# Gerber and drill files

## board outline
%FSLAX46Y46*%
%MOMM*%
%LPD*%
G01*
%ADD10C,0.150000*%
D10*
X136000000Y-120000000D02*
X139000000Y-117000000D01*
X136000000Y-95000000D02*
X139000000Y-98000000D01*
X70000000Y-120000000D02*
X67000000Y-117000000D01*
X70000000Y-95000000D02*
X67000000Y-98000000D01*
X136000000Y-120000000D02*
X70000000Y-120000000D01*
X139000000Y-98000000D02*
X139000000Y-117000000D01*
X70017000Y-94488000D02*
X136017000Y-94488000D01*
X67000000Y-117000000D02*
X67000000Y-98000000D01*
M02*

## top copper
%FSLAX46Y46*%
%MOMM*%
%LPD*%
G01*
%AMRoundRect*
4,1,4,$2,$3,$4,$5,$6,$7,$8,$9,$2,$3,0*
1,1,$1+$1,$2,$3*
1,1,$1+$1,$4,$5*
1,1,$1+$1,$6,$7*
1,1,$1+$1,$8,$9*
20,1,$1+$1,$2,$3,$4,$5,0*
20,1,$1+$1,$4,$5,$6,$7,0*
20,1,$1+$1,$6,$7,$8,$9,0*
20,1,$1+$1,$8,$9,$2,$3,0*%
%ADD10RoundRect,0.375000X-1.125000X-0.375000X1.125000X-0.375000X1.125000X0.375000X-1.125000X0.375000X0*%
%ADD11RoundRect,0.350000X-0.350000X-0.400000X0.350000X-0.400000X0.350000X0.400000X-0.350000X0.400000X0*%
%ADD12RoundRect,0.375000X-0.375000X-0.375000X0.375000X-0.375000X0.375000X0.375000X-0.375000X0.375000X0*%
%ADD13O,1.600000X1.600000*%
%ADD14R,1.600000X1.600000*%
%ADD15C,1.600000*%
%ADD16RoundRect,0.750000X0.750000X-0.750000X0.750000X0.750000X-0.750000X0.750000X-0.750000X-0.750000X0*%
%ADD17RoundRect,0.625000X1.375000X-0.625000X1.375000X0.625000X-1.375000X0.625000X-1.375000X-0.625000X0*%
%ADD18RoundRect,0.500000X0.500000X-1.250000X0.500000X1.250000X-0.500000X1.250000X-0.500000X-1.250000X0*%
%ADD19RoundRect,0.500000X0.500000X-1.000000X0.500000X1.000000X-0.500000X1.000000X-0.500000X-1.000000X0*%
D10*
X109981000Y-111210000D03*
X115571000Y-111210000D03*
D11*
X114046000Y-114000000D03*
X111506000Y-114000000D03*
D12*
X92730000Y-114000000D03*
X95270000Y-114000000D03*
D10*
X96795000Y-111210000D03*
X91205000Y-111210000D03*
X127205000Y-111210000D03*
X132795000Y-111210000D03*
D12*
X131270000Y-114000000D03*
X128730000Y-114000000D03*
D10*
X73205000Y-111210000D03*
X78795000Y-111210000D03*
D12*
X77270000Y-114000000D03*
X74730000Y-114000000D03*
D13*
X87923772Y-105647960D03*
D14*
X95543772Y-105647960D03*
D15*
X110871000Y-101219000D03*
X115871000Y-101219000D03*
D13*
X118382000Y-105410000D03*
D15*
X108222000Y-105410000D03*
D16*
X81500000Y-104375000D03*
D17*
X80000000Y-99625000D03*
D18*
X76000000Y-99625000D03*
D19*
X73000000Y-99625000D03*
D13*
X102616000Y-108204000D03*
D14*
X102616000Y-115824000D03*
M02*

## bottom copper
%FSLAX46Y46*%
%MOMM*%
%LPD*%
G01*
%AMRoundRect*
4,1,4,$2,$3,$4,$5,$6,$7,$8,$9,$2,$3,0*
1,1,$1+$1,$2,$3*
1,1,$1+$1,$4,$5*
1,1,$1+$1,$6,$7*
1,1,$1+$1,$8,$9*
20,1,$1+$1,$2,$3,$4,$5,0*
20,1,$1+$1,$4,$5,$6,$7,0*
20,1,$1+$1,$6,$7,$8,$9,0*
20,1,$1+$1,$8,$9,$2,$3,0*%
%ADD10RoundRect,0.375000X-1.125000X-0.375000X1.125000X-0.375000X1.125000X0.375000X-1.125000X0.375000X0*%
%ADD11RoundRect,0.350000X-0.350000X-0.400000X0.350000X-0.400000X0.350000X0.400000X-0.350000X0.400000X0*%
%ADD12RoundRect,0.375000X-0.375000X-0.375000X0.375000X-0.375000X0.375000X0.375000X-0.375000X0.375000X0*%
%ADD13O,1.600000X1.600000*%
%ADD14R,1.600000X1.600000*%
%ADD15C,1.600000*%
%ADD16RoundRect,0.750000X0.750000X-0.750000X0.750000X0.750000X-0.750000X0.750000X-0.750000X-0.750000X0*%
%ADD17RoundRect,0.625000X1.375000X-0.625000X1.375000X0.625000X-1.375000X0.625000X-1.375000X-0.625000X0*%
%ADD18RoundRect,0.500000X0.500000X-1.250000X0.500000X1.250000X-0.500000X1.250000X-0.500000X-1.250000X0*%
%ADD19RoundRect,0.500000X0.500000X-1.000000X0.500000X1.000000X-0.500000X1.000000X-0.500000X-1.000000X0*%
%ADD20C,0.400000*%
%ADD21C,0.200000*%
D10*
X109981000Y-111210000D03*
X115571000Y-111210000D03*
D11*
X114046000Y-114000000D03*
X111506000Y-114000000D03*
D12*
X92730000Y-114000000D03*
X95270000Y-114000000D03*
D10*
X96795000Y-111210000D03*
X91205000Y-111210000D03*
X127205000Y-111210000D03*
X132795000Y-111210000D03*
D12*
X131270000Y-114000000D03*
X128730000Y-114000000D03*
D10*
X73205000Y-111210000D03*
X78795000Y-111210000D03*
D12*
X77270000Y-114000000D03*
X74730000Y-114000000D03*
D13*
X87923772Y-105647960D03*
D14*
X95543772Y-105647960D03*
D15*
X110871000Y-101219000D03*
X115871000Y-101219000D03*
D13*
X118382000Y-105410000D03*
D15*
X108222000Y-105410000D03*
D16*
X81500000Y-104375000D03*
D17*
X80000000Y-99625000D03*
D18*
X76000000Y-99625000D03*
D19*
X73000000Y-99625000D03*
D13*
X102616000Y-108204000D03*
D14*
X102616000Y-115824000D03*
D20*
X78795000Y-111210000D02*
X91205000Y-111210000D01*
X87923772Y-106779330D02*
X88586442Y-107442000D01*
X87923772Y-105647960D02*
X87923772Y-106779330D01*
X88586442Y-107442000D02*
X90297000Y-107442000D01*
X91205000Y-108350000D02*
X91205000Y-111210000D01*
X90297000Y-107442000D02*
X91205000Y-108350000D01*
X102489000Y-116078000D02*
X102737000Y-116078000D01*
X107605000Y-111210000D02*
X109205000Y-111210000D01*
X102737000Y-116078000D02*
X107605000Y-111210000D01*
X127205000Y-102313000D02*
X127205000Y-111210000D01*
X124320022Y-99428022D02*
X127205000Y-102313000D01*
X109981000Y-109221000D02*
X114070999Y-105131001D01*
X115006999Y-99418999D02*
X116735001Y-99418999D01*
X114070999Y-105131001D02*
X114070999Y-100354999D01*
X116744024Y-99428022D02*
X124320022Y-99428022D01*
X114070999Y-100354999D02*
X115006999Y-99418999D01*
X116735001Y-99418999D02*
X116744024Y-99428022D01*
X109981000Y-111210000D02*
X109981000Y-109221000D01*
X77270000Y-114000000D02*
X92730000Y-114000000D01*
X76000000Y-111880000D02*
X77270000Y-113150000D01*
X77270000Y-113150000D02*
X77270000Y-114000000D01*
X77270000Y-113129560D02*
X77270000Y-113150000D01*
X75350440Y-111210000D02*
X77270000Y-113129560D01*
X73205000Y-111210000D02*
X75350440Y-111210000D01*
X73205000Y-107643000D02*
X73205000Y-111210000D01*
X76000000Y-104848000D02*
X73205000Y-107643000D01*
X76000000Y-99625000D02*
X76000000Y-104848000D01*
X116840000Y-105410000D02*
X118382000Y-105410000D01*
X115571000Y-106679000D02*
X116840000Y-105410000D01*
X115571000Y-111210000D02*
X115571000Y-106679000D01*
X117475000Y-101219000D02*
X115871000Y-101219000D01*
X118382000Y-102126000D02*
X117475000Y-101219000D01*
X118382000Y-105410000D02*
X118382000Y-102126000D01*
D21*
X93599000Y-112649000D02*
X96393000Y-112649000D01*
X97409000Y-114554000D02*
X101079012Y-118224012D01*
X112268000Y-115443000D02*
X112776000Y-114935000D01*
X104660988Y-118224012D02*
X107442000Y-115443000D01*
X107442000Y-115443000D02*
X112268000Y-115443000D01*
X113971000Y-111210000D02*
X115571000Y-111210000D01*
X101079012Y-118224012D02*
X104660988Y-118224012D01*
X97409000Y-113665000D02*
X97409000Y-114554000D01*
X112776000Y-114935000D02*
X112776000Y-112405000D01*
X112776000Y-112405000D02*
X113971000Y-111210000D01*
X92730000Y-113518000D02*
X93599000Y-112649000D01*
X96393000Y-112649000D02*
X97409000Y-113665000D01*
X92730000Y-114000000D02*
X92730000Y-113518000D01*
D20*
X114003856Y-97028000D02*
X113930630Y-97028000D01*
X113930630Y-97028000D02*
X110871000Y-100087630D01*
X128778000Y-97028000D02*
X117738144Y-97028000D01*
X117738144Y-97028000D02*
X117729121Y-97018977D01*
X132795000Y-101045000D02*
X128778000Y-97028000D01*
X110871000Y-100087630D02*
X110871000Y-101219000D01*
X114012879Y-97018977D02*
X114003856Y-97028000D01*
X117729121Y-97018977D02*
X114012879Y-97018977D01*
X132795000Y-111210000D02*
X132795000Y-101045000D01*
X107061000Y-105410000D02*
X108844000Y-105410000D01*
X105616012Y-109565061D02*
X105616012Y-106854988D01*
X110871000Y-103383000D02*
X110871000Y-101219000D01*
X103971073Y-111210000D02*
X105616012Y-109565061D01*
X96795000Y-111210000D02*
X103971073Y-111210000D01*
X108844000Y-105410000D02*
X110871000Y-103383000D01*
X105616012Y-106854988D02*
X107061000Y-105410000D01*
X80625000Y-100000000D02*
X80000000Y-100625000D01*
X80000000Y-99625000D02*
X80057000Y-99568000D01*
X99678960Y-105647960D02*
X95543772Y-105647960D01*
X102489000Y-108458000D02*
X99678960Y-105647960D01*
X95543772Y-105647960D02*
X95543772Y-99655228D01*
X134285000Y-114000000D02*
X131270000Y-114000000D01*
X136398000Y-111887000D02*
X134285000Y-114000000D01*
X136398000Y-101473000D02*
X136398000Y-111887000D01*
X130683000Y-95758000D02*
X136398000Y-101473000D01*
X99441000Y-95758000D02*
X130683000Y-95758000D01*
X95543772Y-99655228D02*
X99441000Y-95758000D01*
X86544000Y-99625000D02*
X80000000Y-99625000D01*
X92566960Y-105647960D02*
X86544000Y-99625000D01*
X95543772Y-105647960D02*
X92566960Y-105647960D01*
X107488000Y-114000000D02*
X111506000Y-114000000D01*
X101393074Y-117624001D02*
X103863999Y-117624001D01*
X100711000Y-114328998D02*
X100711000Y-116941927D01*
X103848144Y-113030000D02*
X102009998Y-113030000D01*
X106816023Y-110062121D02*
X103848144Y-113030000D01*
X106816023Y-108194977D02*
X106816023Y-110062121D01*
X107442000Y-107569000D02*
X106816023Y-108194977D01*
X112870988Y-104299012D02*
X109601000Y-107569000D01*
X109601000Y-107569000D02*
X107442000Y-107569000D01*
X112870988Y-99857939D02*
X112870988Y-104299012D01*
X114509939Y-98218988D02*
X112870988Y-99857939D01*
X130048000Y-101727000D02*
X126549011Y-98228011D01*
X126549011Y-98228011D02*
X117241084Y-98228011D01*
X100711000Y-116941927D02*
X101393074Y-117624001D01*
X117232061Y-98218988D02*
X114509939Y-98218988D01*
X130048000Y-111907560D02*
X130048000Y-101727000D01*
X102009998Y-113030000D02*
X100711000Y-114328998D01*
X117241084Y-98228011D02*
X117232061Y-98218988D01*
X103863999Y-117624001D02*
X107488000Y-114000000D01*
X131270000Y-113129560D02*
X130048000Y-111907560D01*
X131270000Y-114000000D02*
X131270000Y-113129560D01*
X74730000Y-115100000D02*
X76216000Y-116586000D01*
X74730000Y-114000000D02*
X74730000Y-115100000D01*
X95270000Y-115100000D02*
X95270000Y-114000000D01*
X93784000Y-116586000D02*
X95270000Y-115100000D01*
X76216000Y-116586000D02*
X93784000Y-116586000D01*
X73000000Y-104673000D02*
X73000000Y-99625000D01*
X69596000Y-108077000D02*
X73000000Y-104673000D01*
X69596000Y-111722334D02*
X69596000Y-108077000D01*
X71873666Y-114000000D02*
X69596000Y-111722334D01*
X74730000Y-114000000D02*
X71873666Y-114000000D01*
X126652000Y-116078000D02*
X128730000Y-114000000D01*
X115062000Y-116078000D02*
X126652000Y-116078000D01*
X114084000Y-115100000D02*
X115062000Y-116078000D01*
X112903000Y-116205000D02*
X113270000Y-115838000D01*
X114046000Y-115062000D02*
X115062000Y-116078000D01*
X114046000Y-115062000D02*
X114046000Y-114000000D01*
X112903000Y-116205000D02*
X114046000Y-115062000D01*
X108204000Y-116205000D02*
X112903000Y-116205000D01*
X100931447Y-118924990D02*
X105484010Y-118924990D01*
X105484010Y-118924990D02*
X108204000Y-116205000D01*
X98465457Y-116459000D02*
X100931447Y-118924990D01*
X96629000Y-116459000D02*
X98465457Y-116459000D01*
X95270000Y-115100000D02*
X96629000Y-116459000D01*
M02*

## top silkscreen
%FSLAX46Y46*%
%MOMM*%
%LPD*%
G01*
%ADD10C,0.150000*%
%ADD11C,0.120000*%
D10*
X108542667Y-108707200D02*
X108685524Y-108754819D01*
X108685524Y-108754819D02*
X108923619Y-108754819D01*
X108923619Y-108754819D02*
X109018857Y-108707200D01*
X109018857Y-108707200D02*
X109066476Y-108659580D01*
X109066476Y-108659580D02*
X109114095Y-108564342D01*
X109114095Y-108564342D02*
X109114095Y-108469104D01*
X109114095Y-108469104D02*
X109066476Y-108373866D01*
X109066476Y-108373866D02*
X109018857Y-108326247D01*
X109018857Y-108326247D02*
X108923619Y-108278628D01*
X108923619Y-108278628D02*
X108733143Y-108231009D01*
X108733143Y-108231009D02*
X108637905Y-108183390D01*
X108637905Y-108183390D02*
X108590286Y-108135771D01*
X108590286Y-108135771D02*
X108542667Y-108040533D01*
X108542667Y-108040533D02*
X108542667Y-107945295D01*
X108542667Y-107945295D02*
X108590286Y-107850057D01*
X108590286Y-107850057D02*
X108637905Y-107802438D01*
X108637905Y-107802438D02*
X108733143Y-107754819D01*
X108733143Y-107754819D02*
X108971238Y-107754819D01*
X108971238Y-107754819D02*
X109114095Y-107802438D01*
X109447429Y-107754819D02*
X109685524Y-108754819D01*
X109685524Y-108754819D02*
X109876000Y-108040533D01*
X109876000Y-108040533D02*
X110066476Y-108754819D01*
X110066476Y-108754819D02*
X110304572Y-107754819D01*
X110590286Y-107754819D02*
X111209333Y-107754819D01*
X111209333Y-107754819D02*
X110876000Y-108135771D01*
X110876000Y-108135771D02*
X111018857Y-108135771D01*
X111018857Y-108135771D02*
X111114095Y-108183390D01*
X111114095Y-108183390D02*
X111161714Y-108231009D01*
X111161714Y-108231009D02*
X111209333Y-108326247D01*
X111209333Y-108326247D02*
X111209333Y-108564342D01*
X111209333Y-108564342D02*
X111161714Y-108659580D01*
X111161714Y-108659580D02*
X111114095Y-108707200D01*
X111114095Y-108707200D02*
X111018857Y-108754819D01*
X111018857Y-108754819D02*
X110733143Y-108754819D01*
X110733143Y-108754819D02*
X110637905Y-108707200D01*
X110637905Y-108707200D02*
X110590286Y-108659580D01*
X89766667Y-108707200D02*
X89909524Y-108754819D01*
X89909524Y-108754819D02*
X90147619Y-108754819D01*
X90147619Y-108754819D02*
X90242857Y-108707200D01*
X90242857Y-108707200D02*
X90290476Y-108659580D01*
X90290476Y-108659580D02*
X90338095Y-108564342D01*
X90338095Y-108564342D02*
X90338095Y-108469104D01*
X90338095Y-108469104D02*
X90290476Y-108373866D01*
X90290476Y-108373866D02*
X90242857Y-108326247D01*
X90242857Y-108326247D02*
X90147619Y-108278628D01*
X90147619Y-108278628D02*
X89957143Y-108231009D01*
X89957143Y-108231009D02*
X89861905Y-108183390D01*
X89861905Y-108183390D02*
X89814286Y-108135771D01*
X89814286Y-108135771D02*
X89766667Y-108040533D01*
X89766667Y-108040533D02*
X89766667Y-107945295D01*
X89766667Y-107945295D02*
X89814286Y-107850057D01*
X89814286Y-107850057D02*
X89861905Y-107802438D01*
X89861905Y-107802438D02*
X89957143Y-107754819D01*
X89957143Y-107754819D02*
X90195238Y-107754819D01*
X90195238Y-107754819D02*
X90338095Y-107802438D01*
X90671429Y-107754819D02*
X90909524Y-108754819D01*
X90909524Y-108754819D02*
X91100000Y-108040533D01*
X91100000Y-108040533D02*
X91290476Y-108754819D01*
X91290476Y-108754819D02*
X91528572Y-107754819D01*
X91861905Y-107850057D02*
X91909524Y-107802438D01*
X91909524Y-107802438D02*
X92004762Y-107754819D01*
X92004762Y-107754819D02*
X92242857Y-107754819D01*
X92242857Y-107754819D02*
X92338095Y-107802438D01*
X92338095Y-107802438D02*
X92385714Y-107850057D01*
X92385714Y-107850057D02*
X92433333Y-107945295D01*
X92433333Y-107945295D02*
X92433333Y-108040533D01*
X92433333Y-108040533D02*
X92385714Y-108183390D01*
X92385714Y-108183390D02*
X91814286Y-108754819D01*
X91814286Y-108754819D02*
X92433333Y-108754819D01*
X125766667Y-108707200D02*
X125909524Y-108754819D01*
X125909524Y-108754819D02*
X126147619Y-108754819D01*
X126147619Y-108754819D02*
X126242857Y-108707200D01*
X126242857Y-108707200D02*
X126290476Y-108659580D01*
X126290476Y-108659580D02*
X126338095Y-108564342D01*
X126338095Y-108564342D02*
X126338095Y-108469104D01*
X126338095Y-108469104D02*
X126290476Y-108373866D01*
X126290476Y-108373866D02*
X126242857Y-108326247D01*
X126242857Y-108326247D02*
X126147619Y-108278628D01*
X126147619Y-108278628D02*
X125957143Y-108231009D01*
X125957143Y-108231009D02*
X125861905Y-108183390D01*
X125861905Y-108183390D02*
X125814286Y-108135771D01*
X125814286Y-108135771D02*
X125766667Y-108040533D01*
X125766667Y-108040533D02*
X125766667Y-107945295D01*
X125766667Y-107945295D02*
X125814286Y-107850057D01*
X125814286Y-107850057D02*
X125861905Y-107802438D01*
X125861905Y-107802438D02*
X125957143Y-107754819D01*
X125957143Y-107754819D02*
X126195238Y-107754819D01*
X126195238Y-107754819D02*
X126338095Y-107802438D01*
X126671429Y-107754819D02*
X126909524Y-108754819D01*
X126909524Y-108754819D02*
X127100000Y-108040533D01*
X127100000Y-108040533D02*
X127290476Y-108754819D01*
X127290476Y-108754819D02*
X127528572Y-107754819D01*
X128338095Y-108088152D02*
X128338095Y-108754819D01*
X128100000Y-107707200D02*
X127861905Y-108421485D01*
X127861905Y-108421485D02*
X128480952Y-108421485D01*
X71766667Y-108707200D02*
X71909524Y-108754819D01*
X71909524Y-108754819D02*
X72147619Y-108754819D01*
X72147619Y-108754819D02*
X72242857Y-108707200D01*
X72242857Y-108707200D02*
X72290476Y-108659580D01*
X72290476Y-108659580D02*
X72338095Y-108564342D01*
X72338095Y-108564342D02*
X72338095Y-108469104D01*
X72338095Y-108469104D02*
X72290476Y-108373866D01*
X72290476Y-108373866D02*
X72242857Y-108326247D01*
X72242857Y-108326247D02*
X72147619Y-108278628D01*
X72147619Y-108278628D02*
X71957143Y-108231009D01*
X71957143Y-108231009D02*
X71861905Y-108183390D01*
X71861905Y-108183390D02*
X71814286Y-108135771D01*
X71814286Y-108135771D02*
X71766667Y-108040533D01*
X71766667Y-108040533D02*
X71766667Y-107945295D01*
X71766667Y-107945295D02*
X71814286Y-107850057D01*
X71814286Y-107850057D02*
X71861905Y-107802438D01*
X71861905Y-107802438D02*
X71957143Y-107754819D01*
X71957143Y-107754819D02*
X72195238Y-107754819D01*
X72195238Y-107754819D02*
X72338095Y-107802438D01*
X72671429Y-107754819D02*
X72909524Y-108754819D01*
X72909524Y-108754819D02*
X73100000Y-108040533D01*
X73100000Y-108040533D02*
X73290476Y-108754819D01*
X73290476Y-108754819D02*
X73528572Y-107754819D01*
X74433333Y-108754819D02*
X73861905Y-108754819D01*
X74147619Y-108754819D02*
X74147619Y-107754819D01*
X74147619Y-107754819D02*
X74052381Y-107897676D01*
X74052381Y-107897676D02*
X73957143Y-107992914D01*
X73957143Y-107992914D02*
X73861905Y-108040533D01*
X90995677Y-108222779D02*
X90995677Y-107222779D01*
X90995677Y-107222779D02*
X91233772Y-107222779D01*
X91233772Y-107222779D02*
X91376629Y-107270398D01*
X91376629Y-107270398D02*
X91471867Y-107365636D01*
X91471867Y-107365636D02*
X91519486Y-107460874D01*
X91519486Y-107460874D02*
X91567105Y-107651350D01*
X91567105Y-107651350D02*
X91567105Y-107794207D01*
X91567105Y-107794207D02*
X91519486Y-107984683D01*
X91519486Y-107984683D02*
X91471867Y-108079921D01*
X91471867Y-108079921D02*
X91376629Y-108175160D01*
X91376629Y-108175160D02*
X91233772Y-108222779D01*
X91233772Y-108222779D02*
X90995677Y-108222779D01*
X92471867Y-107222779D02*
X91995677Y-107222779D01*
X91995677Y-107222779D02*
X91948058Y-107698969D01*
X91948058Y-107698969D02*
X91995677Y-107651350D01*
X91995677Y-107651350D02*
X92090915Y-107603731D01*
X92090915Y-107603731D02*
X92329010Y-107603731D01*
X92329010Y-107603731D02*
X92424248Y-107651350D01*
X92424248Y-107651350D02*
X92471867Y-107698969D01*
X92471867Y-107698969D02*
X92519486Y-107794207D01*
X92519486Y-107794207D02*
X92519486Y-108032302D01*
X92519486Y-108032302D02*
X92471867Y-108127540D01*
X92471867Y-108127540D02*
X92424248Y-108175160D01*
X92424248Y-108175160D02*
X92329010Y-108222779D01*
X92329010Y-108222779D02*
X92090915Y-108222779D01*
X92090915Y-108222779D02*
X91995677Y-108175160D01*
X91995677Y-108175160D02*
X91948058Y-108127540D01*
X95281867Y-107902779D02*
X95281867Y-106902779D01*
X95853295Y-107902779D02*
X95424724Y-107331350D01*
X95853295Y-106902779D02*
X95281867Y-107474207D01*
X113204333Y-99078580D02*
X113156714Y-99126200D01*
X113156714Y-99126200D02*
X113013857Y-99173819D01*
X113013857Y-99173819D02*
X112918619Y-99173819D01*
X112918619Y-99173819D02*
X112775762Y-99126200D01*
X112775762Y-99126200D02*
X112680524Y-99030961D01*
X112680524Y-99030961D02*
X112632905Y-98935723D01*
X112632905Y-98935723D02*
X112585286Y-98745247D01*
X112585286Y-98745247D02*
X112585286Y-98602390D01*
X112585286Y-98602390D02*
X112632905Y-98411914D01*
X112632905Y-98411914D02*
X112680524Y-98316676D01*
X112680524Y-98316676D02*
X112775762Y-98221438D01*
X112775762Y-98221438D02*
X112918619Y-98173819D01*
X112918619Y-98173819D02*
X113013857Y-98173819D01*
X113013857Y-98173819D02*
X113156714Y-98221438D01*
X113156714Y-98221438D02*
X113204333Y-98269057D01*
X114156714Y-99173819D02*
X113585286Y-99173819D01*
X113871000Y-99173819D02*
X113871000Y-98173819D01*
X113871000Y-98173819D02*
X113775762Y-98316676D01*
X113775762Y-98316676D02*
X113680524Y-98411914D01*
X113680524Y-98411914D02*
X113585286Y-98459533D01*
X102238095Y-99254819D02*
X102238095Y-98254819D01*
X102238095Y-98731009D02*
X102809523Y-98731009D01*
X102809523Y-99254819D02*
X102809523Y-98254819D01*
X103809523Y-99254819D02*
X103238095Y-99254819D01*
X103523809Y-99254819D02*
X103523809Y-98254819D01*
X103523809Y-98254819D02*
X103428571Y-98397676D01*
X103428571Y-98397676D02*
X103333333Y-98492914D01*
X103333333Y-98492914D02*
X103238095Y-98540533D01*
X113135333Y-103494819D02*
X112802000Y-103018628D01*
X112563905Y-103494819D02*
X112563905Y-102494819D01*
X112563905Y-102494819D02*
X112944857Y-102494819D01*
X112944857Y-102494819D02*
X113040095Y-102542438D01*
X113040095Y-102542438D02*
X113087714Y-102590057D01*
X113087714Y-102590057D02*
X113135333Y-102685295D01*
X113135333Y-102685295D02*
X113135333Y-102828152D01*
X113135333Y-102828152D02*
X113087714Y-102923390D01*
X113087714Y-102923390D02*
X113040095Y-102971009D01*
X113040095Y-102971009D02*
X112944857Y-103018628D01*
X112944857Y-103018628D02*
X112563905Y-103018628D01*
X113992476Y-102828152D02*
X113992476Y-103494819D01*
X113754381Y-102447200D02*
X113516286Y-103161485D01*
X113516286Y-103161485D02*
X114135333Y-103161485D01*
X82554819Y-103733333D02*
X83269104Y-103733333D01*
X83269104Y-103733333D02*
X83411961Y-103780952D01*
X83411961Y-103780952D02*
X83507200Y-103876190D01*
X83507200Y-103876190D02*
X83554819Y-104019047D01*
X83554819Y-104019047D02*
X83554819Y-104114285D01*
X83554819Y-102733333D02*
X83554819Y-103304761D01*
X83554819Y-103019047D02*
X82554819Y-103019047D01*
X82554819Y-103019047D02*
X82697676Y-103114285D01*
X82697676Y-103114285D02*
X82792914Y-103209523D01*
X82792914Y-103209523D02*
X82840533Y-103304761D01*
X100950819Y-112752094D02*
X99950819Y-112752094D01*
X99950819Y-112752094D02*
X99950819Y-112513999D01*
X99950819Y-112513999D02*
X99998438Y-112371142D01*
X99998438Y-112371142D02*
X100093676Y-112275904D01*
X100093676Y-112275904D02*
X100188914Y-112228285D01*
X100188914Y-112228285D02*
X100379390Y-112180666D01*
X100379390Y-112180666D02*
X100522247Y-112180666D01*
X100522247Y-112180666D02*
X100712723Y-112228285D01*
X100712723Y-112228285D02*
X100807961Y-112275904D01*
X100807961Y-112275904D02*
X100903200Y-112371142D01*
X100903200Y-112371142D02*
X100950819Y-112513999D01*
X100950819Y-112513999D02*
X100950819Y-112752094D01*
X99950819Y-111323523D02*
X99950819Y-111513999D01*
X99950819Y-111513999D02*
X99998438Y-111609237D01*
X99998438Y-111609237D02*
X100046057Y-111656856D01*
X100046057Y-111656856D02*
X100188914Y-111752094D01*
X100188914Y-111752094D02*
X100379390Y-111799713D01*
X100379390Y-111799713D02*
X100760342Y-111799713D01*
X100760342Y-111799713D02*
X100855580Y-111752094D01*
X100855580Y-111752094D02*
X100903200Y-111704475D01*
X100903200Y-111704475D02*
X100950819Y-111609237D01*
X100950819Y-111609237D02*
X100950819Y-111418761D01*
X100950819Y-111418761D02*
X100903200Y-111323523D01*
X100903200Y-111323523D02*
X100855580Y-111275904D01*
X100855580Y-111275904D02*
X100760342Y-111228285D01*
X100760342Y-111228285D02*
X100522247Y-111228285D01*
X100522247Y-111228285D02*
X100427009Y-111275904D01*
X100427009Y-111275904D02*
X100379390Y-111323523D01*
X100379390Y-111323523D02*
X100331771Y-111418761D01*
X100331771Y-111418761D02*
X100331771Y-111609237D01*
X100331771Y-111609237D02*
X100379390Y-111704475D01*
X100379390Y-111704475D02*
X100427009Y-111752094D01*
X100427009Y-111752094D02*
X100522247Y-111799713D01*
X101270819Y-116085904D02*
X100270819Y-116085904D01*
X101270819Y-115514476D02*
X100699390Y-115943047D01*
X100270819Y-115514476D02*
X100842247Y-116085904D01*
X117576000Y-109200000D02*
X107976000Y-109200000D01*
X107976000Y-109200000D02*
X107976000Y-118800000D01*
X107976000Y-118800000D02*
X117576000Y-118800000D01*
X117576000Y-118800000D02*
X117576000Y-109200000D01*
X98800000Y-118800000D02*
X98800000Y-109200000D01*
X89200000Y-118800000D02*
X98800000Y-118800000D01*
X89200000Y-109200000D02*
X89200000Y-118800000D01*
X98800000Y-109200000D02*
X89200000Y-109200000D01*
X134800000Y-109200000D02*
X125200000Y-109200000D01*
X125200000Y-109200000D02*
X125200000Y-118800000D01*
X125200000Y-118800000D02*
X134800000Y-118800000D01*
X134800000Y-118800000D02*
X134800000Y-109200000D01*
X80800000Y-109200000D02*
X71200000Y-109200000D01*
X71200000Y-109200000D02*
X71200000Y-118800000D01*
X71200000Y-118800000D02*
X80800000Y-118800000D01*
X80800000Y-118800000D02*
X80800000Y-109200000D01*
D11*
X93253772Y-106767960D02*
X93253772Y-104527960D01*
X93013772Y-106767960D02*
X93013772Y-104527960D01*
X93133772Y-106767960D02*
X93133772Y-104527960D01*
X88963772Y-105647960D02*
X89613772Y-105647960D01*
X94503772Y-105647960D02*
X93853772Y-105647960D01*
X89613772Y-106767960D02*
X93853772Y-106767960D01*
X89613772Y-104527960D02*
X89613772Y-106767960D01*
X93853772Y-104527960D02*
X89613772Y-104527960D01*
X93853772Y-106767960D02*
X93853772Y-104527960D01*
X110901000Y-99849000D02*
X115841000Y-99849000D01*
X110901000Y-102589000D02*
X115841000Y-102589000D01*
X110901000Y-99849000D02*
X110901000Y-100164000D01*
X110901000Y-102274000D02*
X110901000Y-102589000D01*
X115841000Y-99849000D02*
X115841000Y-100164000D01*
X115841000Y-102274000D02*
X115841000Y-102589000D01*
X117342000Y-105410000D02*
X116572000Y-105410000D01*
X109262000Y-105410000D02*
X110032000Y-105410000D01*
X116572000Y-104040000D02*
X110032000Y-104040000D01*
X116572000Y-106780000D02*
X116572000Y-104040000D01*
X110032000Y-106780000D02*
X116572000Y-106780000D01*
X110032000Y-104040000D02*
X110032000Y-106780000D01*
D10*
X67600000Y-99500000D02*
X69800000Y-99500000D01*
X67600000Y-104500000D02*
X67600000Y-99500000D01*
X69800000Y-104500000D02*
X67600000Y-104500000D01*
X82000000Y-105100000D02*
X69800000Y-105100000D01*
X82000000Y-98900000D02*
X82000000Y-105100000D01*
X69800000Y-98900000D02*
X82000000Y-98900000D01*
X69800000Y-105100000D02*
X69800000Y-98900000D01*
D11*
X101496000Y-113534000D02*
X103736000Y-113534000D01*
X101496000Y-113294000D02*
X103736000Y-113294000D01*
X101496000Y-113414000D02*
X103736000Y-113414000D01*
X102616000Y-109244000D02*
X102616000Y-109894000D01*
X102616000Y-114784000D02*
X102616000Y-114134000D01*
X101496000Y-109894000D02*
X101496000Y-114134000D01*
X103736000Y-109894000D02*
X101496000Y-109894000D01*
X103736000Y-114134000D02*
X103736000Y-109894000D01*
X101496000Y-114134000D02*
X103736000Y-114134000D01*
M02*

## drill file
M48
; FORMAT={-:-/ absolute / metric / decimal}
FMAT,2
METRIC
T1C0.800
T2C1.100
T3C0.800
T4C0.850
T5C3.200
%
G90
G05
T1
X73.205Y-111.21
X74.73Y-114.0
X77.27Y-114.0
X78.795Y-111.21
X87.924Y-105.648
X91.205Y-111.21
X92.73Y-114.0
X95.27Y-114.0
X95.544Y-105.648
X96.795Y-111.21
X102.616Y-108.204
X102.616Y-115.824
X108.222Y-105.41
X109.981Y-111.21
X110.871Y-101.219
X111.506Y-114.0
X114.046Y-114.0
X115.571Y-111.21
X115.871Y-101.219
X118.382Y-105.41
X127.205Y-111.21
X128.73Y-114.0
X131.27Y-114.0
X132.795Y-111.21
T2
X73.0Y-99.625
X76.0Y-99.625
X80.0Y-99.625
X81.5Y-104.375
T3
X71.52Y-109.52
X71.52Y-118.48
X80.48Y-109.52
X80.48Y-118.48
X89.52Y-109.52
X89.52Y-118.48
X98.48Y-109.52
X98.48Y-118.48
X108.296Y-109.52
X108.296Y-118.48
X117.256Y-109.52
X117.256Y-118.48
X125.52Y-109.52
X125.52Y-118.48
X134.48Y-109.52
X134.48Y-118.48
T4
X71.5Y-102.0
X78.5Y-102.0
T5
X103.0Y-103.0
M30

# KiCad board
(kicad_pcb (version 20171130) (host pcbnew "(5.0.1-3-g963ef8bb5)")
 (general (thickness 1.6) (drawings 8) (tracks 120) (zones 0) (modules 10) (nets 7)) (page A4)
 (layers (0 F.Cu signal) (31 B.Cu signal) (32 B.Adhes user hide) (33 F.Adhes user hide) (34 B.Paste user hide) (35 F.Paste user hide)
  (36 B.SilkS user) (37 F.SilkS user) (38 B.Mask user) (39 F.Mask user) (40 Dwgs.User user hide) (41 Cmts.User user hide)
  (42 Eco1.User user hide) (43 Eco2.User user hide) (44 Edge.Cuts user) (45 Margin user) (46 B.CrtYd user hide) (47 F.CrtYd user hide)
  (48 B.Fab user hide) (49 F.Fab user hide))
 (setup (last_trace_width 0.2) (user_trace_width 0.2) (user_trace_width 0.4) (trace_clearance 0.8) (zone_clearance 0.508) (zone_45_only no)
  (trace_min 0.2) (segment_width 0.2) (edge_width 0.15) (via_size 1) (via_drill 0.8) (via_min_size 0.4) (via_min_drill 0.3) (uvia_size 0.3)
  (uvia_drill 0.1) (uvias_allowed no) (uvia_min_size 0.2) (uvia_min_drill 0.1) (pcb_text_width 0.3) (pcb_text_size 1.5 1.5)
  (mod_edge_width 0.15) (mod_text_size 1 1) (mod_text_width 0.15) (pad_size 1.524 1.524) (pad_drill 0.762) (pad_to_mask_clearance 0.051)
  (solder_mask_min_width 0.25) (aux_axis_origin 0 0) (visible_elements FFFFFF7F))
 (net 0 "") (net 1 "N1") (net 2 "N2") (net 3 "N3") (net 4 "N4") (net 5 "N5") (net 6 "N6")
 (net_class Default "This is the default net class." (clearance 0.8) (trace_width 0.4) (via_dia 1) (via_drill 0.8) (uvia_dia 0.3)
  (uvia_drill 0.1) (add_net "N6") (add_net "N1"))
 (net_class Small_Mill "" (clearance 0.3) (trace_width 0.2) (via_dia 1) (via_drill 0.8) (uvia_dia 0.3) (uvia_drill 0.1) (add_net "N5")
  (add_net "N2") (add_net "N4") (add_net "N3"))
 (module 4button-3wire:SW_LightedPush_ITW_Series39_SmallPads (layer F.Cu) (at 112.776 114)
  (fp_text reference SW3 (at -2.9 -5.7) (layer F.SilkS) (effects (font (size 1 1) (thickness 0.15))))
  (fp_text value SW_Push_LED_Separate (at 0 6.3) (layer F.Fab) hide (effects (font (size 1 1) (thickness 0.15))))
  (fp_line (start 4.8 -4.8) (end -4.8 -4.8) (layer F.SilkS) (width 0.15))
  (fp_line (start -4.8 -4.8) (end -4.8 4.8) (layer F.SilkS) (width 0.15))
  (fp_line (start -4.8 4.8) (end 4.8 4.8) (layer F.SilkS) (width 0.15))
  (fp_line (start 4.8 4.8) (end 4.8 -4.8) (layer F.SilkS) (width 0.15))
  (pad 1 thru_hole roundrect (at -2.795 -2.79) (size 3 1.5) (drill 0.8) (layers *.Cu *.Mask) (roundrect_rratio 0.25) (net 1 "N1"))
  (pad 2 thru_hole roundrect (at 2.795 -2.79) (size 3 1.5) (drill 0.8) (layers *.Cu *.Mask) (roundrect_rratio 0.25) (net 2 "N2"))
  (pad 3 thru_hole roundrect (at 1.27 0) (size 1.4 1.5) (drill 0.8) (layers *.Cu *.Mask) (roundrect_rratio 0.25) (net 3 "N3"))
  (pad 4 thru_hole roundrect (at -1.27 0) (size 1.4 1.5) (drill 0.8) (layers *.Cu *.Mask) (roundrect_rratio 0.25) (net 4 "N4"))
  (pad "" np_thru_hole circle (at 4.48 4.48) (size 0.8 0.8) (drill 0.8) (layers *.Cu *.Mask))
  (pad "" np_thru_hole circle (at -4.48 4.48) (size 0.8 0.8) (drill 0.8) (layers *.Cu *.Mask))
  (pad "" np_thru_hole circle (at 4.48 -4.48) (size 0.8 0.8) (drill 0.8) (layers *.Cu *.Mask))
  (pad "" np_thru_hole circle (at -4.48 -4.48) (size 0.8 0.8) (drill 0.8) (layers *.Cu *.Mask)))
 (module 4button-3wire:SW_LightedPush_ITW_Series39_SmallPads (layer F.Cu) (at 94 114)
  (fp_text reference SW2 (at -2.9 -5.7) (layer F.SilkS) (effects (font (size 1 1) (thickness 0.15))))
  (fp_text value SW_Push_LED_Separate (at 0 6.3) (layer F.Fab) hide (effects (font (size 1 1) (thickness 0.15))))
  (fp_line (start 4.8 4.8) (end 4.8 -4.8) (layer F.SilkS) (width 0.15))
  (fp_line (start -4.8 4.8) (end 4.8 4.8) (layer F.SilkS) (width 0.15))
  (fp_line (start -4.8 -4.8) (end -4.8 4.8) (layer F.SilkS) (width 0.15))
  (fp_line (start 4.8 -4.8) (end -4.8 -4.8) (layer F.SilkS) (width 0.15))
  (pad "" np_thru_hole circle (at -4.48 -4.48) (size 0.8 0.8) (drill 0.8) (layers *.Cu *.Mask))
  (pad "" np_thru_hole circle (at 4.48 -4.48) (size 0.8 0.8) (drill 0.8) (layers *.Cu *.Mask))
  (pad "" np_thru_hole circle (at -4.48 4.48) (size 0.8 0.8) (drill 0.8) (layers *.Cu *.Mask))
  (pad "" np_thru_hole circle (at 4.48 4.48) (size 0.8 0.8) (drill 0.8) (layers *.Cu *.Mask))
  (pad 4 thru_hole roundrect (at -1.27 0) (size 1.5 1.5) (drill 0.8) (layers *.Cu *.Mask) (roundrect_rratio 0.25) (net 2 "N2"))
  (pad 3 thru_hole roundrect (at 1.27 0) (size 1.5 1.5) (drill 0.8) (layers *.Cu *.Mask) (roundrect_rratio 0.25) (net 3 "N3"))
  (pad 2 thru_hole roundrect (at 2.795 -2.79) (size 3 1.5) (drill 0.8) (layers *.Cu *.Mask) (roundrect_rratio 0.25) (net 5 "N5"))
  (pad 1 thru_hole roundrect (at -2.795 -2.79) (size 3 1.5) (drill 0.8) (layers *.Cu *.Mask) (roundrect_rratio 0.25) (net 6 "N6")))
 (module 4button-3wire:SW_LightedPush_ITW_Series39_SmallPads (layer F.Cu) (at 130 114)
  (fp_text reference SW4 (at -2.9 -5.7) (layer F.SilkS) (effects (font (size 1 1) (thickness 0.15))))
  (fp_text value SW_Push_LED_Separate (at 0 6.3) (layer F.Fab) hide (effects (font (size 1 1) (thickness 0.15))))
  (fp_line (start 4.8 -4.8) (end -4.8 -4.8) (layer F.SilkS) (width 0.15))
  (fp_line (start -4.8 -4.8) (end -4.8 4.8) (layer F.SilkS) (width 0.15))
  (fp_line (start -4.8 4.8) (end 4.8 4.8) (layer F.SilkS) (width 0.15))
  (fp_line (start 4.8 4.8) (end 4.8 -4.8) (layer F.SilkS) (width 0.15))
  (pad 1 thru_hole roundrect (at -2.795 -2.79) (size 3 1.5) (drill 0.8) (layers *.Cu *.Mask) (roundrect_rratio 0.25) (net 1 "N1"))
  (pad 2 thru_hole roundrect (at 2.795 -2.79) (size 3 1.5) (drill 0.8) (layers *.Cu *.Mask) (roundrect_rratio 0.25) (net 5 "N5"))
  (pad 3 thru_hole roundrect (at 1.27 0) (size 1.5 1.5) (drill 0.8) (layers *.Cu *.Mask) (roundrect_rratio 0.25) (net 4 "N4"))
  (pad 4 thru_hole roundrect (at -1.27 0) (size 1.5 1.5) (drill 0.8) (layers *.Cu *.Mask) (roundrect_rratio 0.25) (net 3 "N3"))
  (pad "" np_thru_hole circle (at 4.48 4.48) (size 0.8 0.8) (drill 0.8) (layers *.Cu *.Mask))
  (pad "" np_thru_hole circle (at -4.48 4.48) (size 0.8 0.8) (drill 0.8) (layers *.Cu *.Mask))
  (pad "" np_thru_hole circle (at 4.48 -4.48) (size 0.8 0.8) (drill 0.8) (layers *.Cu *.Mask))
  (pad "" np_thru_hole circle (at -4.48 -4.48) (size 0.8 0.8) (drill 0.8) (layers *.Cu *.Mask)))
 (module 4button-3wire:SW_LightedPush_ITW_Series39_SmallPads (layer F.Cu) (at 76 114)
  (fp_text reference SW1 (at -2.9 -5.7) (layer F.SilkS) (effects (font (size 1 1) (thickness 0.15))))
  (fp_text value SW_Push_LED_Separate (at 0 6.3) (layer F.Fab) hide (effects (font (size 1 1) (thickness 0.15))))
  (fp_line (start 4.8 -4.8) (end -4.8 -4.8) (layer F.SilkS) (width 0.15))
  (fp_line (start -4.8 -4.8) (end -4.8 4.8) (layer F.SilkS) (width 0.15))
  (fp_line (start -4.8 4.8) (end 4.8 4.8) (layer F.SilkS) (width 0.15))
  (fp_line (start 4.8 4.8) (end 4.8 -4.8) (layer F.SilkS) (width 0.15))
  (pad 1 thru_hole roundrect (at -2.795 -2.79) (size 3 1.5) (drill 0.8) (layers *.Cu *.Mask) (roundrect_rratio 0.25) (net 2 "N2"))
  (pad 2 thru_hole roundrect (at 2.795 -2.79) (size 3 1.5) (drill 0.8) (layers *.Cu *.Mask) (roundrect_rratio 0.25) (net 6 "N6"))
  (pad 3 thru_hole roundrect (at 1.27 0) (size 1.5 1.5) (drill 0.8) (layers *.Cu *.Mask) (roundrect_rratio 0.25) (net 2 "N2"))
  (pad 4 thru_hole roundrect (at -1.27 0) (size 1.5 1.5) (drill 0.8) (layers *.Cu *.Mask) (roundrect_rratio 0.25) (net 3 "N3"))
  (pad "" np_thru_hole circle (at 4.48 4.48) (size 0.8 0.8) (drill 0.8) (layers *.Cu *.Mask))
  (pad "" np_thru_hole circle (at -4.48 4.48) (size 0.8 0.8) (drill 0.8) (layers *.Cu *.Mask))
  (pad "" np_thru_hole circle (at 4.48 -4.48) (size 0.8 0.8) (drill 0.8) (layers *.Cu *.Mask))
  (pad "" np_thru_hole circle (at -4.48 -4.48) (size 0.8 0.8) (drill 0.8) (layers *.Cu *.Mask)))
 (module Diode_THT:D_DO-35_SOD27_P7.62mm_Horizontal (layer F.Cu) (at 95.543772 105.64796 180)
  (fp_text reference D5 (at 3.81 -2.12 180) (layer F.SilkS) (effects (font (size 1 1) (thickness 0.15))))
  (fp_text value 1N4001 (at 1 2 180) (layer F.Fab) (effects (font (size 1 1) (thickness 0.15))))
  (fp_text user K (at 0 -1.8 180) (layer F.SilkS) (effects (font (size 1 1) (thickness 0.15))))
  (fp_line (start 2.29 -1.12) (end 2.29 1.12) (layer F.SilkS) (width 0.12))
  (fp_line (start 2.53 -1.12) (end 2.53 1.12) (layer F.SilkS) (width 0.12))
  (fp_line (start 2.41 -1.12) (end 2.41 1.12) (layer F.SilkS) (width 0.12))
  (fp_line (start 6.58 0) (end 5.93 0) (layer F.SilkS) (width 0.12))
  (fp_line (start 1.04 0) (end 1.69 0) (layer F.SilkS) (width 0.12))
  (fp_line (start 5.93 -1.12) (end 1.69 -1.12) (layer F.SilkS) (width 0.12))
  (fp_line (start 5.93 1.12) (end 5.93 -1.12) (layer F.SilkS) (width 0.12))
  (fp_line (start 1.69 1.12) (end 5.93 1.12) (layer F.SilkS) (width 0.12))
  (fp_line (start 1.69 -1.12) (end 1.69 1.12) (layer F.SilkS) (width 0.12))
  (pad 2 thru_hole oval (at 7.62 0 180) (size 1.6 1.6) (drill 0.8) (layers *.Cu *.Mask) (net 6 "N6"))
  (pad 1 thru_hole rect (at 0 0 180) (size 1.6 1.6) (drill 0.8) (layers *.Cu *.Mask) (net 4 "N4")))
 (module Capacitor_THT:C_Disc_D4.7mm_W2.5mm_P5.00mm (layer F.Cu) (at 110.871 101.219)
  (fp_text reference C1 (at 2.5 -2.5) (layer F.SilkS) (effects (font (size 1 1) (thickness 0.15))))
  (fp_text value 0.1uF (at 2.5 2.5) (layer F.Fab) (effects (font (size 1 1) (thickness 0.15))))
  (fp_line (start 0.03 -1.37) (end 4.97 -1.37) (layer F.SilkS) (width 0.12))
  (fp_line (start 0.03 1.37) (end 4.97 1.37) (layer F.SilkS) (width 0.12))
  (fp_line (start 0.03 -1.37) (end 0.03 -1.055) (layer F.SilkS) (width 0.12))
  (fp_line (start 0.03 1.055) (end 0.03 1.37) (layer F.SilkS) (width 0.12))
  (fp_line (start 4.97 -1.37) (end 4.97 -1.055) (layer F.SilkS) (width 0.12))
  (fp_line (start 4.97 1.055) (end 4.97 1.37) (layer F.SilkS) (width 0.12))
  (pad 1 thru_hole circle (at 0 0) (size 1.6 1.6) (drill 0.8) (layers *.Cu *.Mask) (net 5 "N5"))
  (pad 2 thru_hole circle (at 5 0) (size 1.6 1.6) (drill 0.8) (layers *.Cu *.Mask) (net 2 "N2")))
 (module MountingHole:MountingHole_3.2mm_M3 (layer F.Cu) (at 103 103)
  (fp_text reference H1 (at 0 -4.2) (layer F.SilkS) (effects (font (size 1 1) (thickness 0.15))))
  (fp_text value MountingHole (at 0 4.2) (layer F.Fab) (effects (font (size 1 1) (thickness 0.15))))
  (pad 1 np_thru_hole circle (at 0 0) (size 3.2 3.2) (drill 3.2) (layers *.Cu *.Mask)))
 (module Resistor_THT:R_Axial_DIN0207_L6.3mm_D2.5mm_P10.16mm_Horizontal (layer F.Cu) (at 108.222 105.41)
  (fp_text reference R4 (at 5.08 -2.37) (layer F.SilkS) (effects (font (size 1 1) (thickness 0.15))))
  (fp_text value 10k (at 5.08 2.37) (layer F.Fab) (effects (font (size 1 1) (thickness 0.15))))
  (fp_line (start 9.12 0) (end 8.35 0) (layer F.SilkS) (width 0.12))
  (fp_line (start 1.04 0) (end 1.81 0) (layer F.SilkS) (width 0.12))
  (fp_line (start 8.35 -1.37) (end 1.81 -1.37) (layer F.SilkS) (width 0.12))
  (fp_line (start 8.35 1.37) (end 8.35 -1.37) (layer F.SilkS) (width 0.12))
  (fp_line (start 1.81 1.37) (end 8.35 1.37) (layer F.SilkS) (width 0.12))
  (fp_line (start 1.81 -1.37) (end 1.81 1.37) (layer F.SilkS) (width 0.12))
  (pad 2 thru_hole oval (at 10.16 0) (size 1.6 1.6) (drill 0.8) (layers *.Cu *.Mask) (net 2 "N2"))
  (pad 1 thru_hole circle (at 0 0) (size 1.6 1.6) (drill 0.8) (layers *.Cu *.Mask) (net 5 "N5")))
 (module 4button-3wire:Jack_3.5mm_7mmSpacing (layer F.Cu) (at 82 102 90)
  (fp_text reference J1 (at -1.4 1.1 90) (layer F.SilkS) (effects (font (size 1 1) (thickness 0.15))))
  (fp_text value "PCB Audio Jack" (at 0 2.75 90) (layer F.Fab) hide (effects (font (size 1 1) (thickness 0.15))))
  (fp_line (start 2.5 -14.4) (end 2.5 -12.2) (layer F.SilkS) (width 0.15))
  (fp_line (start -2.5 -14.4) (end 2.5 -14.4) (layer F.SilkS) (width 0.15))
  (fp_line (start -2.5 -12.2) (end -2.5 -14.4) (layer F.SilkS) (width 0.15))
  (fp_line (start -3.1 0) (end -3.1 -12.2) (layer F.SilkS) (width 0.15))
  (fp_line (start 3.1 0) (end -3.1 0) (layer F.SilkS) (width 0.15))
  (fp_line (start 3.1 -12.2) (end 3.1 0) (layer F.SilkS) (width 0.15))
  (fp_line (start -3.1 -12.2) (end 3.1 -12.2) (layer F.SilkS) (width 0.15))
  (pad "" np_thru_hole circle (at 0 -3.5 90) (size 0.85 0.85) (drill 0.85) (layers *.Cu *.Mask))
  (pad "" np_thru_hole circle (at 0 -10.5 90) (size 0.85 0.85) (drill 0.85) (layers *.Cu *.Mask))
  (pad X thru_hole roundrect (at -2.375 -0.5 90) (size 3 3) (drill 1.1) (layers *.Cu *.Mask) (roundrect_rratio 0.25))
  (pad T thru_hole roundrect (at 2.375 -2 90) (size 2.5 4) (drill 1.1) (layers *.Cu *.Mask) (roundrect_rratio 0.25) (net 4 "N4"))
  (pad R thru_hole roundrect (at 2.375 -6 90) (size 3.5 2) (drill 1.1) (layers *.Cu *.Mask) (roundrect_rratio 0.25) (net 2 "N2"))
  (pad S thru_hole roundrect (at 2.375 -9 90) (size 3 2) (drill 1.1) (layers *.Cu *.Mask) (roundrect_rratio 0.25) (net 3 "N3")))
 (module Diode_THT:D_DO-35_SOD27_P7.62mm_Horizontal (layer F.Cu) (at 102.616 115.824 90)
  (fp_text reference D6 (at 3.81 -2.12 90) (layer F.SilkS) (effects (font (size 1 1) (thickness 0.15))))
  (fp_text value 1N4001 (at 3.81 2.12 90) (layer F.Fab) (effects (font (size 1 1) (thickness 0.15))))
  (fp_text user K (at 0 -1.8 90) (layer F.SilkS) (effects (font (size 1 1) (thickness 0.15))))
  (fp_line (start 2.29 -1.12) (end 2.29 1.12) (layer F.SilkS) (width 0.12))
  (fp_line (start 2.53 -1.12) (end 2.53 1.12) (layer F.SilkS) (width 0.12))
  (fp_line (start 2.41 -1.12) (end 2.41 1.12) (layer F.SilkS) (width 0.12))
  (fp_line (start 6.58 0) (end 5.93 0) (layer F.SilkS) (width 0.12))
  (fp_line (start 1.04 0) (end 1.69 0) (layer F.SilkS) (width 0.12))
  (fp_line (start 5.93 -1.12) (end 1.69 -1.12) (layer F.SilkS) (width 0.12))
  (fp_line (start 5.93 1.12) (end 5.93 -1.12) (layer F.SilkS) (width 0.12))
  (fp_line (start 1.69 1.12) (end 5.93 1.12) (layer F.SilkS) (width 0.12))
  (fp_line (start 1.69 -1.12) (end 1.69 1.12) (layer F.SilkS) (width 0.12))
  (pad 2 thru_hole oval (at 7.62 0 90) (size 1.6 1.6) (drill 0.8) (layers *.Cu *.Mask) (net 4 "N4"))
  (pad 1 thru_hole rect (at 0 0 90) (size 1.6 1.6) (drill 0.8) (layers *.Cu *.Mask) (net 1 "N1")))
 (gr_line (start 136 120) (end 139 117) (layer Edge.Cuts) (width 0.15))
 (gr_line (start 136 95) (end 139 98) (layer Edge.Cuts) (width 0.15))
 (gr_line (start 70 120) (end 67 117) (layer Edge.Cuts) (width 0.15))
 (gr_line (start 70 95) (end 67 98) (layer Edge.Cuts) (width 0.15))
 (gr_line (start 136 120) (end 70 120) (layer Edge.Cuts) (width 0.15))
 (gr_line (start 139 98) (end 139 117) (layer Edge.Cuts) (width 0.15))
 (gr_line (start 70.017 94.488) (end 136.017 94.488) (layer Edge.Cuts) (width 0.15))
 (gr_line (start 67 117) (end 67 98) (layer Edge.Cuts) (width 0.15))
 (segment (start 78.795 111.21) (end 91.205 111.21) (width 0.4) (layer B.Cu) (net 6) (status 30))
 (segment (start 87.923772 106.77933) (end 88.586442 107.442) (width 0.4) (layer B.Cu) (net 6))
 (segment (start 87.923772 105.64796) (end 87.923772 106.77933) (width 0.4) (layer B.Cu) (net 6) (status 10))
 (segment (start 88.586442 107.442) (end 90.297 107.442) (width 0.4) (layer B.Cu) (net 6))
 (segment (start 91.205 108.35) (end 91.205 111.21) (width 0.4) (layer B.Cu) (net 6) (status 20))
 (segment (start 90.297 107.442) (end 91.205 108.35) (width 0.4) (layer B.Cu) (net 6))
 (segment (start 102.489 116.078) (end 102.737 116.078) (width 0.4) (layer B.Cu) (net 1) (status 30))
 (segment (start 107.605 111.21) (end 109.205 111.21) (width 0.4) (layer B.Cu) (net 1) (status 20))
 (segment (start 102.737 116.078) (end 107.605 111.21) (width 0.4) (layer B.Cu) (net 1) (status 10))
 (segment (start 127.205 102.313) (end 127.205 111.21) (width 0.4) (layer B.Cu) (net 1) (status 20))
 (segment (start 124.320022 99.428022) (end 127.205 102.313) (width 0.4) (layer B.Cu) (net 1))
 (segment (start 109.981 109.221) (end 114.070999 105.131001) (width 0.4) (layer B.Cu) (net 1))
 (segment (start 115.006999 99.418999) (end 116.735001 99.418999) (width 0.4) (layer B.Cu) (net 1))
 (segment (start 114.070999 105.131001) (end 114.070999 100.354999) (width 0.4) (layer B.Cu) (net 1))
 (segment (start 116.744024 99.428022) (end 124.320022 99.428022) (width 0.4) (layer B.Cu) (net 1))
 (segment (start 114.070999 100.354999) (end 115.006999 99.418999) (width 0.4) (layer B.Cu) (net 1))
 (segment (start 116.735001 99.418999) (end 116.744024 99.428022) (width 0.4) (layer B.Cu) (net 1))
 (segment (start 109.981 111.21) (end 109.981 109.221) (width 0.4) (layer B.Cu) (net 1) (status 10))
 (segment (start 77.27 114) (end 92.73 114) (width 0.4) (layer B.Cu) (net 2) (status 30))
 (segment (start 76 111.88) (end 77.27 113.15) (width 0.4) (layer B.Cu) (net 2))
 (segment (start 77.27 113.15) (end 77.27 114) (width 0.4) (layer B.Cu) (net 2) (status 20))
 (segment (start 77.27 113.12956) (end 77.27 113.15) (width 0.4) (layer B.Cu) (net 2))
 (segment (start 75.35044 111.21) (end 77.27 113.12956) (width 0.4) (layer B.Cu) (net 2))
 (segment (start 73.205 111.21) (end 75.35044 111.21) (width 0.4) (layer B.Cu) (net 2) (status 10))
 (segment (start 73.205 107.643) (end 73.205 111.21) (width 0.4) (layer B.Cu) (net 2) (status 20))
 (segment (start 76 104.848) (end 73.205 107.643) (width 0.4) (layer B.Cu) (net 2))
 (segment (start 76 99.625) (end 76 104.848) (width 0.4) (layer B.Cu) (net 2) (status 10))
 (segment (start 116.84 105.41) (end 118.382 105.41) (width 0.4) (layer B.Cu) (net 2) (status 20))
 (segment (start 115.571 106.679) (end 116.84 105.41) (width 0.4) (layer B.Cu) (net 2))
 (segment (start 115.571 111.21) (end 115.571 106.679) (width 0.4) (layer B.Cu) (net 2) (status 10))
 (segment (start 117.475 101.219) (end 115.871 101.219) (width 0.4) (layer B.Cu) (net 2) (status 20))
 (segment (start 118.382 102.126) (end 117.475 101.219) (width 0.4) (layer B.Cu) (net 2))
 (segment (start 118.382 105.41) (end 118.382 102.126) (width 0.4) (layer B.Cu) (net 2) (status 10))
 (segment (start 93.599 112.649) (end 96.393 112.649) (width 0.2) (layer B.Cu) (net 2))
 (segment (start 97.409 114.554) (end 101.079012 118.224012) (width 0.2) (layer B.Cu) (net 2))
 (segment (start 112.268 115.443) (end 112.776 114.935) (width 0.2) (layer B.Cu) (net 2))
 (segment (start 104.660988 118.224012) (end 107.442 115.443) (width 0.2) (layer B.Cu) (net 2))
 (segment (start 107.442 115.443) (end 112.268 115.443) (width 0.2) (layer B.Cu) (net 2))
 (segment (start 113.971 111.21) (end 115.571 111.21) (width 0.2) (layer B.Cu) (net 2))
 (segment (start 101.079012 118.224012) (end 104.660988 118.224012) (width 0.2) (layer B.Cu) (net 2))
 (segment (start 97.409 113.665) (end 97.409 114.554) (width 0.2) (layer B.Cu) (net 2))
 (segment (start 112.776 114.935) (end 112.776 112.405) (width 0.2) (layer B.Cu) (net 2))
 (segment (start 112.776 112.405) (end 113.971 111.21) (width 0.2) (layer B.Cu) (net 2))
 (segment (start 92.73 113.518) (end 93.599 112.649) (width 0.2) (layer B.Cu) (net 2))
 (segment (start 96.393 112.649) (end 97.409 113.665) (width 0.2) (layer B.Cu) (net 2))
 (segment (start 92.73 114) (end 92.73 113.518) (width 0.2) (layer B.Cu) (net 2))
 (segment (start 114.003856 97.028) (end 113.93063 97.028) (width 0.4) (layer B.Cu) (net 5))
 (segment (start 113.93063 97.028) (end 110.871 100.08763) (width 0.4) (layer B.Cu) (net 5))
 (segment (start 128.778 97.028) (end 117.738144 97.028) (width 0.4) (layer B.Cu) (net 5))
 (segment (start 117.738144 97.028) (end 117.729121 97.018977) (width 0.4) (layer B.Cu) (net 5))
 (segment (start 132.795 101.045) (end 128.778 97.028) (width 0.4) (layer B.Cu) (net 5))
 (segment (start 110.871 100.08763) (end 110.871 101.219) (width 0.4) (layer B.Cu) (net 5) (status 20))
 (segment (start 114.012879 97.018977) (end 114.003856 97.028) (width 0.4) (layer B.Cu) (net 5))
 (segment (start 117.729121 97.018977) (end 114.012879 97.018977) (width 0.4) (layer B.Cu) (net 5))
 (segment (start 132.795 111.21) (end 132.795 101.045) (width 0.4) (layer B.Cu) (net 5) (status 10))
 (segment (start 107.061 105.41) (end 108.844 105.41) (width 0.4) (layer B.Cu) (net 5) (status 20))
 (segment (start 105.616012 109.565061) (end 105.616012 106.854988) (width 0.4) (layer B.Cu) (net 5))
 (segment (start 110.871 103.383) (end 110.871 101.219) (width 0.4) (layer B.Cu) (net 5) (status 20))
 (segment (start 103.971073 111.21) (end 105.616012 109.565061) (width 0.4) (layer B.Cu) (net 5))
 (segment (start 96.795 111.21) (end 103.971073 111.21) (width 0.4) (layer B.Cu) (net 5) (status 10))
 (segment (start 108.844 105.41) (end 110.871 103.383) (width 0.4) (layer B.Cu) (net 5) (status 10))
 (segment (start 105.616012 106.854988) (end 107.061 105.41) (width 0.4) (layer B.Cu) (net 5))
 (segment (start 80.625 100) (end 80 100.625) (width 0.4) (layer B.Cu) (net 4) (status 30))
 (segment (start 80 99.625) (end 80.057 99.568) (width 0.4) (layer B.Cu) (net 4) (status 30))
 (segment (start 99.67896 105.64796) (end 95.543772 105.64796) (width 0.4) (layer B.Cu) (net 4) (status 20))
 (segment (start 102.489 108.458) (end 99.67896 105.64796) (width 0.4) (layer B.Cu) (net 4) (status 10))
 (segment (start 95.543772 105.64796) (end 95.543772 99.655228) (width 0.4) (layer B.Cu) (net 4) (status 10))
 (segment (start 134.285 114) (end 131.27 114) (width 0.4) (layer B.Cu) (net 4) (status 20))
 (segment (start 136.398 111.887) (end 134.285 114) (width 0.4) (layer B.Cu) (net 4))
 (segment (start 136.398 101.473) (end 136.398 111.887) (width 0.4) (layer B.Cu) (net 4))
 (segment (start 130.683 95.758) (end 136.398 101.473) (width 0.4) (layer B.Cu) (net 4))
 (segment (start 99.441 95.758) (end 130.683 95.758) (width 0.4) (layer B.Cu) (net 4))
 (segment (start 95.543772 99.655228) (end 99.441 95.758) (width 0.4) (layer B.Cu) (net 4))
 (segment (start 86.544 99.625) (end 80 99.625) (width 0.4) (layer B.Cu) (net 4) (status 20))
 (segment (start 92.56696 105.64796) (end 86.544 99.625) (width 0.4) (layer B.Cu) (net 4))
 (segment (start 95.543772 105.64796) (end 92.56696 105.64796) (width 0.4) (layer B.Cu) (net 4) (status 10))
 (segment (start 107.488 114) (end 111.506 114) (width 0.4) (layer B.Cu) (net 4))
 (segment (start 101.393074 117.624001) (end 103.863999 117.624001) (width 0.4) (layer B.Cu) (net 4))
 (segment (start 100.711 114.328998) (end 100.711 116.941927) (width 0.4) (layer B.Cu) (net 4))
 (segment (start 103.848144 113.03) (end 102.009998 113.03) (width 0.4) (layer B.Cu) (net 4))
 (segment (start 106.816023 110.062121) (end 103.848144 113.03) (width 0.4) (layer B.Cu) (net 4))
 (segment (start 106.816023 108.194977) (end 106.816023 110.062121) (width 0.4) (layer B.Cu) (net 4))
 (segment (start 107.442 107.569) (end 106.816023 108.194977) (width 0.4) (layer B.Cu) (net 4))
 (segment (start 112.870988 104.299012) (end 109.601 107.569) (width 0.4) (layer B.Cu) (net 4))
 (segment (start 109.601 107.569) (end 107.442 107.569) (width 0.4) (layer B.Cu) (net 4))
 (segment (start 112.870988 99.857939) (end 112.870988 104.299012) (width 0.4) (layer B.Cu) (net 4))
 (segment (start 114.509939 98.218988) (end 112.870988 99.857939) (width 0.4) (layer B.Cu) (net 4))
 (segment (start 130.048 101.727) (end 126.549011 98.228011) (width 0.4) (layer B.Cu) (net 4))
 (segment (start 126.549011 98.228011) (end 117.241084 98.228011) (width 0.4) (layer B.Cu) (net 4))
 (segment (start 100.711 116.941927) (end 101.393074 117.624001) (width 0.4) (layer B.Cu) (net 4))
 (segment (start 117.232061 98.218988) (end 114.509939 98.218988) (width 0.4) (layer B.Cu) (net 4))
 (segment (start 130.048 111.90756) (end 130.048 101.727) (width 0.4) (layer B.Cu) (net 4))
 (segment (start 102.009998 113.03) (end 100.711 114.328998) (width 0.4) (layer B.Cu) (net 4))
 (segment (start 117.241084 98.228011) (end 117.232061 98.218988) (width 0.4) (layer B.Cu) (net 4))
 (segment (start 103.863999 117.624001) (end 107.488 114) (width 0.4) (layer B.Cu) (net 4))
 (segment (start 131.27 113.12956) (end 130.048 111.90756) (width 0.4) (layer B.Cu) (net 4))
 (segment (start 131.27 114) (end 131.27 113.12956) (width 0.4) (layer B.Cu) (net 4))
 (segment (start 74.73 115.1) (end 76.216 116.586) (width 0.4) (layer B.Cu) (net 3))
 (segment (start 74.73 114) (end 74.73 115.1) (width 0.4) (layer B.Cu) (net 3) (status 10))
 (segment (start 95.27 115.1) (end 95.27 114) (width 0.4) (layer B.Cu) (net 3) (status 20))
 (segment (start 93.784 116.586) (end 95.27 115.1) (width 0.4) (layer B.Cu) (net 3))
 (segment (start 76.216 116.586) (end 93.784 116.586) (width 0.4) (layer B.Cu) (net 3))
 (segment (start 73 104.673) (end 73 99.625) (width 0.4) (layer B.Cu) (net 3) (status 20))
 (segment (start 69.596 108.077) (end 73 104.673) (width 0.4) (layer B.Cu) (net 3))
 (segment (start 69.596 111.722334) (end 69.596 108.077) (width 0.4) (layer B.Cu) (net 3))
 (segment (start 71.873666 114) (end 69.596 111.722334) (width 0.4) (layer B.Cu) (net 3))
 (segment (start 74.73 114) (end 71.873666 114) (width 0.4) (layer B.Cu) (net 3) (status 10))
 (segment (start 126.652 116.078) (end 128.73 114) (width 0.4) (layer B.Cu) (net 3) (status 20))
 (segment (start 115.062 116.078) (end 126.652 116.078) (width 0.4) (layer B.Cu) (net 3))
 (segment (start 114.084 115.1) (end 115.062 116.078) (width 0.4) (layer B.Cu) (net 3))
 (segment (start 112.903 116.205) (end 113.27 115.838) (width 0.4) (layer B.Cu) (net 3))
 (segment (start 114.046 115.062) (end 115.062 116.078) (width 0.4) (layer B.Cu) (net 3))
 (segment (start 114.046 115.062) (end 114.046 114) (width 0.4) (layer B.Cu) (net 3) (status 20))
 (segment (start 112.903 116.205) (end 114.046 115.062) (width 0.4) (layer B.Cu) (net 3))
 (segment (start 108.204 116.205) (end 112.903 116.205) (width 0.4) (layer B.Cu) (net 3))
 (segment (start 100.931447 118.92499) (end 105.48401 118.92499) (width 0.4) (layer B.Cu) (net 3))
 (segment (start 105.48401 118.92499) (end 108.204 116.205) (width 0.4) (layer B.Cu) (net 3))
 (segment (start 98.465457 116.459) (end 100.931447 118.92499) (width 0.4) (layer B.Cu) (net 3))
 (segment (start 96.629 116.459) (end 98.465457 116.459) (width 0.4) (layer B.Cu) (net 3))
 (segment (start 95.27 115.1) (end 96.629 116.459) (width 0.4) (layer B.Cu) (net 3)))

